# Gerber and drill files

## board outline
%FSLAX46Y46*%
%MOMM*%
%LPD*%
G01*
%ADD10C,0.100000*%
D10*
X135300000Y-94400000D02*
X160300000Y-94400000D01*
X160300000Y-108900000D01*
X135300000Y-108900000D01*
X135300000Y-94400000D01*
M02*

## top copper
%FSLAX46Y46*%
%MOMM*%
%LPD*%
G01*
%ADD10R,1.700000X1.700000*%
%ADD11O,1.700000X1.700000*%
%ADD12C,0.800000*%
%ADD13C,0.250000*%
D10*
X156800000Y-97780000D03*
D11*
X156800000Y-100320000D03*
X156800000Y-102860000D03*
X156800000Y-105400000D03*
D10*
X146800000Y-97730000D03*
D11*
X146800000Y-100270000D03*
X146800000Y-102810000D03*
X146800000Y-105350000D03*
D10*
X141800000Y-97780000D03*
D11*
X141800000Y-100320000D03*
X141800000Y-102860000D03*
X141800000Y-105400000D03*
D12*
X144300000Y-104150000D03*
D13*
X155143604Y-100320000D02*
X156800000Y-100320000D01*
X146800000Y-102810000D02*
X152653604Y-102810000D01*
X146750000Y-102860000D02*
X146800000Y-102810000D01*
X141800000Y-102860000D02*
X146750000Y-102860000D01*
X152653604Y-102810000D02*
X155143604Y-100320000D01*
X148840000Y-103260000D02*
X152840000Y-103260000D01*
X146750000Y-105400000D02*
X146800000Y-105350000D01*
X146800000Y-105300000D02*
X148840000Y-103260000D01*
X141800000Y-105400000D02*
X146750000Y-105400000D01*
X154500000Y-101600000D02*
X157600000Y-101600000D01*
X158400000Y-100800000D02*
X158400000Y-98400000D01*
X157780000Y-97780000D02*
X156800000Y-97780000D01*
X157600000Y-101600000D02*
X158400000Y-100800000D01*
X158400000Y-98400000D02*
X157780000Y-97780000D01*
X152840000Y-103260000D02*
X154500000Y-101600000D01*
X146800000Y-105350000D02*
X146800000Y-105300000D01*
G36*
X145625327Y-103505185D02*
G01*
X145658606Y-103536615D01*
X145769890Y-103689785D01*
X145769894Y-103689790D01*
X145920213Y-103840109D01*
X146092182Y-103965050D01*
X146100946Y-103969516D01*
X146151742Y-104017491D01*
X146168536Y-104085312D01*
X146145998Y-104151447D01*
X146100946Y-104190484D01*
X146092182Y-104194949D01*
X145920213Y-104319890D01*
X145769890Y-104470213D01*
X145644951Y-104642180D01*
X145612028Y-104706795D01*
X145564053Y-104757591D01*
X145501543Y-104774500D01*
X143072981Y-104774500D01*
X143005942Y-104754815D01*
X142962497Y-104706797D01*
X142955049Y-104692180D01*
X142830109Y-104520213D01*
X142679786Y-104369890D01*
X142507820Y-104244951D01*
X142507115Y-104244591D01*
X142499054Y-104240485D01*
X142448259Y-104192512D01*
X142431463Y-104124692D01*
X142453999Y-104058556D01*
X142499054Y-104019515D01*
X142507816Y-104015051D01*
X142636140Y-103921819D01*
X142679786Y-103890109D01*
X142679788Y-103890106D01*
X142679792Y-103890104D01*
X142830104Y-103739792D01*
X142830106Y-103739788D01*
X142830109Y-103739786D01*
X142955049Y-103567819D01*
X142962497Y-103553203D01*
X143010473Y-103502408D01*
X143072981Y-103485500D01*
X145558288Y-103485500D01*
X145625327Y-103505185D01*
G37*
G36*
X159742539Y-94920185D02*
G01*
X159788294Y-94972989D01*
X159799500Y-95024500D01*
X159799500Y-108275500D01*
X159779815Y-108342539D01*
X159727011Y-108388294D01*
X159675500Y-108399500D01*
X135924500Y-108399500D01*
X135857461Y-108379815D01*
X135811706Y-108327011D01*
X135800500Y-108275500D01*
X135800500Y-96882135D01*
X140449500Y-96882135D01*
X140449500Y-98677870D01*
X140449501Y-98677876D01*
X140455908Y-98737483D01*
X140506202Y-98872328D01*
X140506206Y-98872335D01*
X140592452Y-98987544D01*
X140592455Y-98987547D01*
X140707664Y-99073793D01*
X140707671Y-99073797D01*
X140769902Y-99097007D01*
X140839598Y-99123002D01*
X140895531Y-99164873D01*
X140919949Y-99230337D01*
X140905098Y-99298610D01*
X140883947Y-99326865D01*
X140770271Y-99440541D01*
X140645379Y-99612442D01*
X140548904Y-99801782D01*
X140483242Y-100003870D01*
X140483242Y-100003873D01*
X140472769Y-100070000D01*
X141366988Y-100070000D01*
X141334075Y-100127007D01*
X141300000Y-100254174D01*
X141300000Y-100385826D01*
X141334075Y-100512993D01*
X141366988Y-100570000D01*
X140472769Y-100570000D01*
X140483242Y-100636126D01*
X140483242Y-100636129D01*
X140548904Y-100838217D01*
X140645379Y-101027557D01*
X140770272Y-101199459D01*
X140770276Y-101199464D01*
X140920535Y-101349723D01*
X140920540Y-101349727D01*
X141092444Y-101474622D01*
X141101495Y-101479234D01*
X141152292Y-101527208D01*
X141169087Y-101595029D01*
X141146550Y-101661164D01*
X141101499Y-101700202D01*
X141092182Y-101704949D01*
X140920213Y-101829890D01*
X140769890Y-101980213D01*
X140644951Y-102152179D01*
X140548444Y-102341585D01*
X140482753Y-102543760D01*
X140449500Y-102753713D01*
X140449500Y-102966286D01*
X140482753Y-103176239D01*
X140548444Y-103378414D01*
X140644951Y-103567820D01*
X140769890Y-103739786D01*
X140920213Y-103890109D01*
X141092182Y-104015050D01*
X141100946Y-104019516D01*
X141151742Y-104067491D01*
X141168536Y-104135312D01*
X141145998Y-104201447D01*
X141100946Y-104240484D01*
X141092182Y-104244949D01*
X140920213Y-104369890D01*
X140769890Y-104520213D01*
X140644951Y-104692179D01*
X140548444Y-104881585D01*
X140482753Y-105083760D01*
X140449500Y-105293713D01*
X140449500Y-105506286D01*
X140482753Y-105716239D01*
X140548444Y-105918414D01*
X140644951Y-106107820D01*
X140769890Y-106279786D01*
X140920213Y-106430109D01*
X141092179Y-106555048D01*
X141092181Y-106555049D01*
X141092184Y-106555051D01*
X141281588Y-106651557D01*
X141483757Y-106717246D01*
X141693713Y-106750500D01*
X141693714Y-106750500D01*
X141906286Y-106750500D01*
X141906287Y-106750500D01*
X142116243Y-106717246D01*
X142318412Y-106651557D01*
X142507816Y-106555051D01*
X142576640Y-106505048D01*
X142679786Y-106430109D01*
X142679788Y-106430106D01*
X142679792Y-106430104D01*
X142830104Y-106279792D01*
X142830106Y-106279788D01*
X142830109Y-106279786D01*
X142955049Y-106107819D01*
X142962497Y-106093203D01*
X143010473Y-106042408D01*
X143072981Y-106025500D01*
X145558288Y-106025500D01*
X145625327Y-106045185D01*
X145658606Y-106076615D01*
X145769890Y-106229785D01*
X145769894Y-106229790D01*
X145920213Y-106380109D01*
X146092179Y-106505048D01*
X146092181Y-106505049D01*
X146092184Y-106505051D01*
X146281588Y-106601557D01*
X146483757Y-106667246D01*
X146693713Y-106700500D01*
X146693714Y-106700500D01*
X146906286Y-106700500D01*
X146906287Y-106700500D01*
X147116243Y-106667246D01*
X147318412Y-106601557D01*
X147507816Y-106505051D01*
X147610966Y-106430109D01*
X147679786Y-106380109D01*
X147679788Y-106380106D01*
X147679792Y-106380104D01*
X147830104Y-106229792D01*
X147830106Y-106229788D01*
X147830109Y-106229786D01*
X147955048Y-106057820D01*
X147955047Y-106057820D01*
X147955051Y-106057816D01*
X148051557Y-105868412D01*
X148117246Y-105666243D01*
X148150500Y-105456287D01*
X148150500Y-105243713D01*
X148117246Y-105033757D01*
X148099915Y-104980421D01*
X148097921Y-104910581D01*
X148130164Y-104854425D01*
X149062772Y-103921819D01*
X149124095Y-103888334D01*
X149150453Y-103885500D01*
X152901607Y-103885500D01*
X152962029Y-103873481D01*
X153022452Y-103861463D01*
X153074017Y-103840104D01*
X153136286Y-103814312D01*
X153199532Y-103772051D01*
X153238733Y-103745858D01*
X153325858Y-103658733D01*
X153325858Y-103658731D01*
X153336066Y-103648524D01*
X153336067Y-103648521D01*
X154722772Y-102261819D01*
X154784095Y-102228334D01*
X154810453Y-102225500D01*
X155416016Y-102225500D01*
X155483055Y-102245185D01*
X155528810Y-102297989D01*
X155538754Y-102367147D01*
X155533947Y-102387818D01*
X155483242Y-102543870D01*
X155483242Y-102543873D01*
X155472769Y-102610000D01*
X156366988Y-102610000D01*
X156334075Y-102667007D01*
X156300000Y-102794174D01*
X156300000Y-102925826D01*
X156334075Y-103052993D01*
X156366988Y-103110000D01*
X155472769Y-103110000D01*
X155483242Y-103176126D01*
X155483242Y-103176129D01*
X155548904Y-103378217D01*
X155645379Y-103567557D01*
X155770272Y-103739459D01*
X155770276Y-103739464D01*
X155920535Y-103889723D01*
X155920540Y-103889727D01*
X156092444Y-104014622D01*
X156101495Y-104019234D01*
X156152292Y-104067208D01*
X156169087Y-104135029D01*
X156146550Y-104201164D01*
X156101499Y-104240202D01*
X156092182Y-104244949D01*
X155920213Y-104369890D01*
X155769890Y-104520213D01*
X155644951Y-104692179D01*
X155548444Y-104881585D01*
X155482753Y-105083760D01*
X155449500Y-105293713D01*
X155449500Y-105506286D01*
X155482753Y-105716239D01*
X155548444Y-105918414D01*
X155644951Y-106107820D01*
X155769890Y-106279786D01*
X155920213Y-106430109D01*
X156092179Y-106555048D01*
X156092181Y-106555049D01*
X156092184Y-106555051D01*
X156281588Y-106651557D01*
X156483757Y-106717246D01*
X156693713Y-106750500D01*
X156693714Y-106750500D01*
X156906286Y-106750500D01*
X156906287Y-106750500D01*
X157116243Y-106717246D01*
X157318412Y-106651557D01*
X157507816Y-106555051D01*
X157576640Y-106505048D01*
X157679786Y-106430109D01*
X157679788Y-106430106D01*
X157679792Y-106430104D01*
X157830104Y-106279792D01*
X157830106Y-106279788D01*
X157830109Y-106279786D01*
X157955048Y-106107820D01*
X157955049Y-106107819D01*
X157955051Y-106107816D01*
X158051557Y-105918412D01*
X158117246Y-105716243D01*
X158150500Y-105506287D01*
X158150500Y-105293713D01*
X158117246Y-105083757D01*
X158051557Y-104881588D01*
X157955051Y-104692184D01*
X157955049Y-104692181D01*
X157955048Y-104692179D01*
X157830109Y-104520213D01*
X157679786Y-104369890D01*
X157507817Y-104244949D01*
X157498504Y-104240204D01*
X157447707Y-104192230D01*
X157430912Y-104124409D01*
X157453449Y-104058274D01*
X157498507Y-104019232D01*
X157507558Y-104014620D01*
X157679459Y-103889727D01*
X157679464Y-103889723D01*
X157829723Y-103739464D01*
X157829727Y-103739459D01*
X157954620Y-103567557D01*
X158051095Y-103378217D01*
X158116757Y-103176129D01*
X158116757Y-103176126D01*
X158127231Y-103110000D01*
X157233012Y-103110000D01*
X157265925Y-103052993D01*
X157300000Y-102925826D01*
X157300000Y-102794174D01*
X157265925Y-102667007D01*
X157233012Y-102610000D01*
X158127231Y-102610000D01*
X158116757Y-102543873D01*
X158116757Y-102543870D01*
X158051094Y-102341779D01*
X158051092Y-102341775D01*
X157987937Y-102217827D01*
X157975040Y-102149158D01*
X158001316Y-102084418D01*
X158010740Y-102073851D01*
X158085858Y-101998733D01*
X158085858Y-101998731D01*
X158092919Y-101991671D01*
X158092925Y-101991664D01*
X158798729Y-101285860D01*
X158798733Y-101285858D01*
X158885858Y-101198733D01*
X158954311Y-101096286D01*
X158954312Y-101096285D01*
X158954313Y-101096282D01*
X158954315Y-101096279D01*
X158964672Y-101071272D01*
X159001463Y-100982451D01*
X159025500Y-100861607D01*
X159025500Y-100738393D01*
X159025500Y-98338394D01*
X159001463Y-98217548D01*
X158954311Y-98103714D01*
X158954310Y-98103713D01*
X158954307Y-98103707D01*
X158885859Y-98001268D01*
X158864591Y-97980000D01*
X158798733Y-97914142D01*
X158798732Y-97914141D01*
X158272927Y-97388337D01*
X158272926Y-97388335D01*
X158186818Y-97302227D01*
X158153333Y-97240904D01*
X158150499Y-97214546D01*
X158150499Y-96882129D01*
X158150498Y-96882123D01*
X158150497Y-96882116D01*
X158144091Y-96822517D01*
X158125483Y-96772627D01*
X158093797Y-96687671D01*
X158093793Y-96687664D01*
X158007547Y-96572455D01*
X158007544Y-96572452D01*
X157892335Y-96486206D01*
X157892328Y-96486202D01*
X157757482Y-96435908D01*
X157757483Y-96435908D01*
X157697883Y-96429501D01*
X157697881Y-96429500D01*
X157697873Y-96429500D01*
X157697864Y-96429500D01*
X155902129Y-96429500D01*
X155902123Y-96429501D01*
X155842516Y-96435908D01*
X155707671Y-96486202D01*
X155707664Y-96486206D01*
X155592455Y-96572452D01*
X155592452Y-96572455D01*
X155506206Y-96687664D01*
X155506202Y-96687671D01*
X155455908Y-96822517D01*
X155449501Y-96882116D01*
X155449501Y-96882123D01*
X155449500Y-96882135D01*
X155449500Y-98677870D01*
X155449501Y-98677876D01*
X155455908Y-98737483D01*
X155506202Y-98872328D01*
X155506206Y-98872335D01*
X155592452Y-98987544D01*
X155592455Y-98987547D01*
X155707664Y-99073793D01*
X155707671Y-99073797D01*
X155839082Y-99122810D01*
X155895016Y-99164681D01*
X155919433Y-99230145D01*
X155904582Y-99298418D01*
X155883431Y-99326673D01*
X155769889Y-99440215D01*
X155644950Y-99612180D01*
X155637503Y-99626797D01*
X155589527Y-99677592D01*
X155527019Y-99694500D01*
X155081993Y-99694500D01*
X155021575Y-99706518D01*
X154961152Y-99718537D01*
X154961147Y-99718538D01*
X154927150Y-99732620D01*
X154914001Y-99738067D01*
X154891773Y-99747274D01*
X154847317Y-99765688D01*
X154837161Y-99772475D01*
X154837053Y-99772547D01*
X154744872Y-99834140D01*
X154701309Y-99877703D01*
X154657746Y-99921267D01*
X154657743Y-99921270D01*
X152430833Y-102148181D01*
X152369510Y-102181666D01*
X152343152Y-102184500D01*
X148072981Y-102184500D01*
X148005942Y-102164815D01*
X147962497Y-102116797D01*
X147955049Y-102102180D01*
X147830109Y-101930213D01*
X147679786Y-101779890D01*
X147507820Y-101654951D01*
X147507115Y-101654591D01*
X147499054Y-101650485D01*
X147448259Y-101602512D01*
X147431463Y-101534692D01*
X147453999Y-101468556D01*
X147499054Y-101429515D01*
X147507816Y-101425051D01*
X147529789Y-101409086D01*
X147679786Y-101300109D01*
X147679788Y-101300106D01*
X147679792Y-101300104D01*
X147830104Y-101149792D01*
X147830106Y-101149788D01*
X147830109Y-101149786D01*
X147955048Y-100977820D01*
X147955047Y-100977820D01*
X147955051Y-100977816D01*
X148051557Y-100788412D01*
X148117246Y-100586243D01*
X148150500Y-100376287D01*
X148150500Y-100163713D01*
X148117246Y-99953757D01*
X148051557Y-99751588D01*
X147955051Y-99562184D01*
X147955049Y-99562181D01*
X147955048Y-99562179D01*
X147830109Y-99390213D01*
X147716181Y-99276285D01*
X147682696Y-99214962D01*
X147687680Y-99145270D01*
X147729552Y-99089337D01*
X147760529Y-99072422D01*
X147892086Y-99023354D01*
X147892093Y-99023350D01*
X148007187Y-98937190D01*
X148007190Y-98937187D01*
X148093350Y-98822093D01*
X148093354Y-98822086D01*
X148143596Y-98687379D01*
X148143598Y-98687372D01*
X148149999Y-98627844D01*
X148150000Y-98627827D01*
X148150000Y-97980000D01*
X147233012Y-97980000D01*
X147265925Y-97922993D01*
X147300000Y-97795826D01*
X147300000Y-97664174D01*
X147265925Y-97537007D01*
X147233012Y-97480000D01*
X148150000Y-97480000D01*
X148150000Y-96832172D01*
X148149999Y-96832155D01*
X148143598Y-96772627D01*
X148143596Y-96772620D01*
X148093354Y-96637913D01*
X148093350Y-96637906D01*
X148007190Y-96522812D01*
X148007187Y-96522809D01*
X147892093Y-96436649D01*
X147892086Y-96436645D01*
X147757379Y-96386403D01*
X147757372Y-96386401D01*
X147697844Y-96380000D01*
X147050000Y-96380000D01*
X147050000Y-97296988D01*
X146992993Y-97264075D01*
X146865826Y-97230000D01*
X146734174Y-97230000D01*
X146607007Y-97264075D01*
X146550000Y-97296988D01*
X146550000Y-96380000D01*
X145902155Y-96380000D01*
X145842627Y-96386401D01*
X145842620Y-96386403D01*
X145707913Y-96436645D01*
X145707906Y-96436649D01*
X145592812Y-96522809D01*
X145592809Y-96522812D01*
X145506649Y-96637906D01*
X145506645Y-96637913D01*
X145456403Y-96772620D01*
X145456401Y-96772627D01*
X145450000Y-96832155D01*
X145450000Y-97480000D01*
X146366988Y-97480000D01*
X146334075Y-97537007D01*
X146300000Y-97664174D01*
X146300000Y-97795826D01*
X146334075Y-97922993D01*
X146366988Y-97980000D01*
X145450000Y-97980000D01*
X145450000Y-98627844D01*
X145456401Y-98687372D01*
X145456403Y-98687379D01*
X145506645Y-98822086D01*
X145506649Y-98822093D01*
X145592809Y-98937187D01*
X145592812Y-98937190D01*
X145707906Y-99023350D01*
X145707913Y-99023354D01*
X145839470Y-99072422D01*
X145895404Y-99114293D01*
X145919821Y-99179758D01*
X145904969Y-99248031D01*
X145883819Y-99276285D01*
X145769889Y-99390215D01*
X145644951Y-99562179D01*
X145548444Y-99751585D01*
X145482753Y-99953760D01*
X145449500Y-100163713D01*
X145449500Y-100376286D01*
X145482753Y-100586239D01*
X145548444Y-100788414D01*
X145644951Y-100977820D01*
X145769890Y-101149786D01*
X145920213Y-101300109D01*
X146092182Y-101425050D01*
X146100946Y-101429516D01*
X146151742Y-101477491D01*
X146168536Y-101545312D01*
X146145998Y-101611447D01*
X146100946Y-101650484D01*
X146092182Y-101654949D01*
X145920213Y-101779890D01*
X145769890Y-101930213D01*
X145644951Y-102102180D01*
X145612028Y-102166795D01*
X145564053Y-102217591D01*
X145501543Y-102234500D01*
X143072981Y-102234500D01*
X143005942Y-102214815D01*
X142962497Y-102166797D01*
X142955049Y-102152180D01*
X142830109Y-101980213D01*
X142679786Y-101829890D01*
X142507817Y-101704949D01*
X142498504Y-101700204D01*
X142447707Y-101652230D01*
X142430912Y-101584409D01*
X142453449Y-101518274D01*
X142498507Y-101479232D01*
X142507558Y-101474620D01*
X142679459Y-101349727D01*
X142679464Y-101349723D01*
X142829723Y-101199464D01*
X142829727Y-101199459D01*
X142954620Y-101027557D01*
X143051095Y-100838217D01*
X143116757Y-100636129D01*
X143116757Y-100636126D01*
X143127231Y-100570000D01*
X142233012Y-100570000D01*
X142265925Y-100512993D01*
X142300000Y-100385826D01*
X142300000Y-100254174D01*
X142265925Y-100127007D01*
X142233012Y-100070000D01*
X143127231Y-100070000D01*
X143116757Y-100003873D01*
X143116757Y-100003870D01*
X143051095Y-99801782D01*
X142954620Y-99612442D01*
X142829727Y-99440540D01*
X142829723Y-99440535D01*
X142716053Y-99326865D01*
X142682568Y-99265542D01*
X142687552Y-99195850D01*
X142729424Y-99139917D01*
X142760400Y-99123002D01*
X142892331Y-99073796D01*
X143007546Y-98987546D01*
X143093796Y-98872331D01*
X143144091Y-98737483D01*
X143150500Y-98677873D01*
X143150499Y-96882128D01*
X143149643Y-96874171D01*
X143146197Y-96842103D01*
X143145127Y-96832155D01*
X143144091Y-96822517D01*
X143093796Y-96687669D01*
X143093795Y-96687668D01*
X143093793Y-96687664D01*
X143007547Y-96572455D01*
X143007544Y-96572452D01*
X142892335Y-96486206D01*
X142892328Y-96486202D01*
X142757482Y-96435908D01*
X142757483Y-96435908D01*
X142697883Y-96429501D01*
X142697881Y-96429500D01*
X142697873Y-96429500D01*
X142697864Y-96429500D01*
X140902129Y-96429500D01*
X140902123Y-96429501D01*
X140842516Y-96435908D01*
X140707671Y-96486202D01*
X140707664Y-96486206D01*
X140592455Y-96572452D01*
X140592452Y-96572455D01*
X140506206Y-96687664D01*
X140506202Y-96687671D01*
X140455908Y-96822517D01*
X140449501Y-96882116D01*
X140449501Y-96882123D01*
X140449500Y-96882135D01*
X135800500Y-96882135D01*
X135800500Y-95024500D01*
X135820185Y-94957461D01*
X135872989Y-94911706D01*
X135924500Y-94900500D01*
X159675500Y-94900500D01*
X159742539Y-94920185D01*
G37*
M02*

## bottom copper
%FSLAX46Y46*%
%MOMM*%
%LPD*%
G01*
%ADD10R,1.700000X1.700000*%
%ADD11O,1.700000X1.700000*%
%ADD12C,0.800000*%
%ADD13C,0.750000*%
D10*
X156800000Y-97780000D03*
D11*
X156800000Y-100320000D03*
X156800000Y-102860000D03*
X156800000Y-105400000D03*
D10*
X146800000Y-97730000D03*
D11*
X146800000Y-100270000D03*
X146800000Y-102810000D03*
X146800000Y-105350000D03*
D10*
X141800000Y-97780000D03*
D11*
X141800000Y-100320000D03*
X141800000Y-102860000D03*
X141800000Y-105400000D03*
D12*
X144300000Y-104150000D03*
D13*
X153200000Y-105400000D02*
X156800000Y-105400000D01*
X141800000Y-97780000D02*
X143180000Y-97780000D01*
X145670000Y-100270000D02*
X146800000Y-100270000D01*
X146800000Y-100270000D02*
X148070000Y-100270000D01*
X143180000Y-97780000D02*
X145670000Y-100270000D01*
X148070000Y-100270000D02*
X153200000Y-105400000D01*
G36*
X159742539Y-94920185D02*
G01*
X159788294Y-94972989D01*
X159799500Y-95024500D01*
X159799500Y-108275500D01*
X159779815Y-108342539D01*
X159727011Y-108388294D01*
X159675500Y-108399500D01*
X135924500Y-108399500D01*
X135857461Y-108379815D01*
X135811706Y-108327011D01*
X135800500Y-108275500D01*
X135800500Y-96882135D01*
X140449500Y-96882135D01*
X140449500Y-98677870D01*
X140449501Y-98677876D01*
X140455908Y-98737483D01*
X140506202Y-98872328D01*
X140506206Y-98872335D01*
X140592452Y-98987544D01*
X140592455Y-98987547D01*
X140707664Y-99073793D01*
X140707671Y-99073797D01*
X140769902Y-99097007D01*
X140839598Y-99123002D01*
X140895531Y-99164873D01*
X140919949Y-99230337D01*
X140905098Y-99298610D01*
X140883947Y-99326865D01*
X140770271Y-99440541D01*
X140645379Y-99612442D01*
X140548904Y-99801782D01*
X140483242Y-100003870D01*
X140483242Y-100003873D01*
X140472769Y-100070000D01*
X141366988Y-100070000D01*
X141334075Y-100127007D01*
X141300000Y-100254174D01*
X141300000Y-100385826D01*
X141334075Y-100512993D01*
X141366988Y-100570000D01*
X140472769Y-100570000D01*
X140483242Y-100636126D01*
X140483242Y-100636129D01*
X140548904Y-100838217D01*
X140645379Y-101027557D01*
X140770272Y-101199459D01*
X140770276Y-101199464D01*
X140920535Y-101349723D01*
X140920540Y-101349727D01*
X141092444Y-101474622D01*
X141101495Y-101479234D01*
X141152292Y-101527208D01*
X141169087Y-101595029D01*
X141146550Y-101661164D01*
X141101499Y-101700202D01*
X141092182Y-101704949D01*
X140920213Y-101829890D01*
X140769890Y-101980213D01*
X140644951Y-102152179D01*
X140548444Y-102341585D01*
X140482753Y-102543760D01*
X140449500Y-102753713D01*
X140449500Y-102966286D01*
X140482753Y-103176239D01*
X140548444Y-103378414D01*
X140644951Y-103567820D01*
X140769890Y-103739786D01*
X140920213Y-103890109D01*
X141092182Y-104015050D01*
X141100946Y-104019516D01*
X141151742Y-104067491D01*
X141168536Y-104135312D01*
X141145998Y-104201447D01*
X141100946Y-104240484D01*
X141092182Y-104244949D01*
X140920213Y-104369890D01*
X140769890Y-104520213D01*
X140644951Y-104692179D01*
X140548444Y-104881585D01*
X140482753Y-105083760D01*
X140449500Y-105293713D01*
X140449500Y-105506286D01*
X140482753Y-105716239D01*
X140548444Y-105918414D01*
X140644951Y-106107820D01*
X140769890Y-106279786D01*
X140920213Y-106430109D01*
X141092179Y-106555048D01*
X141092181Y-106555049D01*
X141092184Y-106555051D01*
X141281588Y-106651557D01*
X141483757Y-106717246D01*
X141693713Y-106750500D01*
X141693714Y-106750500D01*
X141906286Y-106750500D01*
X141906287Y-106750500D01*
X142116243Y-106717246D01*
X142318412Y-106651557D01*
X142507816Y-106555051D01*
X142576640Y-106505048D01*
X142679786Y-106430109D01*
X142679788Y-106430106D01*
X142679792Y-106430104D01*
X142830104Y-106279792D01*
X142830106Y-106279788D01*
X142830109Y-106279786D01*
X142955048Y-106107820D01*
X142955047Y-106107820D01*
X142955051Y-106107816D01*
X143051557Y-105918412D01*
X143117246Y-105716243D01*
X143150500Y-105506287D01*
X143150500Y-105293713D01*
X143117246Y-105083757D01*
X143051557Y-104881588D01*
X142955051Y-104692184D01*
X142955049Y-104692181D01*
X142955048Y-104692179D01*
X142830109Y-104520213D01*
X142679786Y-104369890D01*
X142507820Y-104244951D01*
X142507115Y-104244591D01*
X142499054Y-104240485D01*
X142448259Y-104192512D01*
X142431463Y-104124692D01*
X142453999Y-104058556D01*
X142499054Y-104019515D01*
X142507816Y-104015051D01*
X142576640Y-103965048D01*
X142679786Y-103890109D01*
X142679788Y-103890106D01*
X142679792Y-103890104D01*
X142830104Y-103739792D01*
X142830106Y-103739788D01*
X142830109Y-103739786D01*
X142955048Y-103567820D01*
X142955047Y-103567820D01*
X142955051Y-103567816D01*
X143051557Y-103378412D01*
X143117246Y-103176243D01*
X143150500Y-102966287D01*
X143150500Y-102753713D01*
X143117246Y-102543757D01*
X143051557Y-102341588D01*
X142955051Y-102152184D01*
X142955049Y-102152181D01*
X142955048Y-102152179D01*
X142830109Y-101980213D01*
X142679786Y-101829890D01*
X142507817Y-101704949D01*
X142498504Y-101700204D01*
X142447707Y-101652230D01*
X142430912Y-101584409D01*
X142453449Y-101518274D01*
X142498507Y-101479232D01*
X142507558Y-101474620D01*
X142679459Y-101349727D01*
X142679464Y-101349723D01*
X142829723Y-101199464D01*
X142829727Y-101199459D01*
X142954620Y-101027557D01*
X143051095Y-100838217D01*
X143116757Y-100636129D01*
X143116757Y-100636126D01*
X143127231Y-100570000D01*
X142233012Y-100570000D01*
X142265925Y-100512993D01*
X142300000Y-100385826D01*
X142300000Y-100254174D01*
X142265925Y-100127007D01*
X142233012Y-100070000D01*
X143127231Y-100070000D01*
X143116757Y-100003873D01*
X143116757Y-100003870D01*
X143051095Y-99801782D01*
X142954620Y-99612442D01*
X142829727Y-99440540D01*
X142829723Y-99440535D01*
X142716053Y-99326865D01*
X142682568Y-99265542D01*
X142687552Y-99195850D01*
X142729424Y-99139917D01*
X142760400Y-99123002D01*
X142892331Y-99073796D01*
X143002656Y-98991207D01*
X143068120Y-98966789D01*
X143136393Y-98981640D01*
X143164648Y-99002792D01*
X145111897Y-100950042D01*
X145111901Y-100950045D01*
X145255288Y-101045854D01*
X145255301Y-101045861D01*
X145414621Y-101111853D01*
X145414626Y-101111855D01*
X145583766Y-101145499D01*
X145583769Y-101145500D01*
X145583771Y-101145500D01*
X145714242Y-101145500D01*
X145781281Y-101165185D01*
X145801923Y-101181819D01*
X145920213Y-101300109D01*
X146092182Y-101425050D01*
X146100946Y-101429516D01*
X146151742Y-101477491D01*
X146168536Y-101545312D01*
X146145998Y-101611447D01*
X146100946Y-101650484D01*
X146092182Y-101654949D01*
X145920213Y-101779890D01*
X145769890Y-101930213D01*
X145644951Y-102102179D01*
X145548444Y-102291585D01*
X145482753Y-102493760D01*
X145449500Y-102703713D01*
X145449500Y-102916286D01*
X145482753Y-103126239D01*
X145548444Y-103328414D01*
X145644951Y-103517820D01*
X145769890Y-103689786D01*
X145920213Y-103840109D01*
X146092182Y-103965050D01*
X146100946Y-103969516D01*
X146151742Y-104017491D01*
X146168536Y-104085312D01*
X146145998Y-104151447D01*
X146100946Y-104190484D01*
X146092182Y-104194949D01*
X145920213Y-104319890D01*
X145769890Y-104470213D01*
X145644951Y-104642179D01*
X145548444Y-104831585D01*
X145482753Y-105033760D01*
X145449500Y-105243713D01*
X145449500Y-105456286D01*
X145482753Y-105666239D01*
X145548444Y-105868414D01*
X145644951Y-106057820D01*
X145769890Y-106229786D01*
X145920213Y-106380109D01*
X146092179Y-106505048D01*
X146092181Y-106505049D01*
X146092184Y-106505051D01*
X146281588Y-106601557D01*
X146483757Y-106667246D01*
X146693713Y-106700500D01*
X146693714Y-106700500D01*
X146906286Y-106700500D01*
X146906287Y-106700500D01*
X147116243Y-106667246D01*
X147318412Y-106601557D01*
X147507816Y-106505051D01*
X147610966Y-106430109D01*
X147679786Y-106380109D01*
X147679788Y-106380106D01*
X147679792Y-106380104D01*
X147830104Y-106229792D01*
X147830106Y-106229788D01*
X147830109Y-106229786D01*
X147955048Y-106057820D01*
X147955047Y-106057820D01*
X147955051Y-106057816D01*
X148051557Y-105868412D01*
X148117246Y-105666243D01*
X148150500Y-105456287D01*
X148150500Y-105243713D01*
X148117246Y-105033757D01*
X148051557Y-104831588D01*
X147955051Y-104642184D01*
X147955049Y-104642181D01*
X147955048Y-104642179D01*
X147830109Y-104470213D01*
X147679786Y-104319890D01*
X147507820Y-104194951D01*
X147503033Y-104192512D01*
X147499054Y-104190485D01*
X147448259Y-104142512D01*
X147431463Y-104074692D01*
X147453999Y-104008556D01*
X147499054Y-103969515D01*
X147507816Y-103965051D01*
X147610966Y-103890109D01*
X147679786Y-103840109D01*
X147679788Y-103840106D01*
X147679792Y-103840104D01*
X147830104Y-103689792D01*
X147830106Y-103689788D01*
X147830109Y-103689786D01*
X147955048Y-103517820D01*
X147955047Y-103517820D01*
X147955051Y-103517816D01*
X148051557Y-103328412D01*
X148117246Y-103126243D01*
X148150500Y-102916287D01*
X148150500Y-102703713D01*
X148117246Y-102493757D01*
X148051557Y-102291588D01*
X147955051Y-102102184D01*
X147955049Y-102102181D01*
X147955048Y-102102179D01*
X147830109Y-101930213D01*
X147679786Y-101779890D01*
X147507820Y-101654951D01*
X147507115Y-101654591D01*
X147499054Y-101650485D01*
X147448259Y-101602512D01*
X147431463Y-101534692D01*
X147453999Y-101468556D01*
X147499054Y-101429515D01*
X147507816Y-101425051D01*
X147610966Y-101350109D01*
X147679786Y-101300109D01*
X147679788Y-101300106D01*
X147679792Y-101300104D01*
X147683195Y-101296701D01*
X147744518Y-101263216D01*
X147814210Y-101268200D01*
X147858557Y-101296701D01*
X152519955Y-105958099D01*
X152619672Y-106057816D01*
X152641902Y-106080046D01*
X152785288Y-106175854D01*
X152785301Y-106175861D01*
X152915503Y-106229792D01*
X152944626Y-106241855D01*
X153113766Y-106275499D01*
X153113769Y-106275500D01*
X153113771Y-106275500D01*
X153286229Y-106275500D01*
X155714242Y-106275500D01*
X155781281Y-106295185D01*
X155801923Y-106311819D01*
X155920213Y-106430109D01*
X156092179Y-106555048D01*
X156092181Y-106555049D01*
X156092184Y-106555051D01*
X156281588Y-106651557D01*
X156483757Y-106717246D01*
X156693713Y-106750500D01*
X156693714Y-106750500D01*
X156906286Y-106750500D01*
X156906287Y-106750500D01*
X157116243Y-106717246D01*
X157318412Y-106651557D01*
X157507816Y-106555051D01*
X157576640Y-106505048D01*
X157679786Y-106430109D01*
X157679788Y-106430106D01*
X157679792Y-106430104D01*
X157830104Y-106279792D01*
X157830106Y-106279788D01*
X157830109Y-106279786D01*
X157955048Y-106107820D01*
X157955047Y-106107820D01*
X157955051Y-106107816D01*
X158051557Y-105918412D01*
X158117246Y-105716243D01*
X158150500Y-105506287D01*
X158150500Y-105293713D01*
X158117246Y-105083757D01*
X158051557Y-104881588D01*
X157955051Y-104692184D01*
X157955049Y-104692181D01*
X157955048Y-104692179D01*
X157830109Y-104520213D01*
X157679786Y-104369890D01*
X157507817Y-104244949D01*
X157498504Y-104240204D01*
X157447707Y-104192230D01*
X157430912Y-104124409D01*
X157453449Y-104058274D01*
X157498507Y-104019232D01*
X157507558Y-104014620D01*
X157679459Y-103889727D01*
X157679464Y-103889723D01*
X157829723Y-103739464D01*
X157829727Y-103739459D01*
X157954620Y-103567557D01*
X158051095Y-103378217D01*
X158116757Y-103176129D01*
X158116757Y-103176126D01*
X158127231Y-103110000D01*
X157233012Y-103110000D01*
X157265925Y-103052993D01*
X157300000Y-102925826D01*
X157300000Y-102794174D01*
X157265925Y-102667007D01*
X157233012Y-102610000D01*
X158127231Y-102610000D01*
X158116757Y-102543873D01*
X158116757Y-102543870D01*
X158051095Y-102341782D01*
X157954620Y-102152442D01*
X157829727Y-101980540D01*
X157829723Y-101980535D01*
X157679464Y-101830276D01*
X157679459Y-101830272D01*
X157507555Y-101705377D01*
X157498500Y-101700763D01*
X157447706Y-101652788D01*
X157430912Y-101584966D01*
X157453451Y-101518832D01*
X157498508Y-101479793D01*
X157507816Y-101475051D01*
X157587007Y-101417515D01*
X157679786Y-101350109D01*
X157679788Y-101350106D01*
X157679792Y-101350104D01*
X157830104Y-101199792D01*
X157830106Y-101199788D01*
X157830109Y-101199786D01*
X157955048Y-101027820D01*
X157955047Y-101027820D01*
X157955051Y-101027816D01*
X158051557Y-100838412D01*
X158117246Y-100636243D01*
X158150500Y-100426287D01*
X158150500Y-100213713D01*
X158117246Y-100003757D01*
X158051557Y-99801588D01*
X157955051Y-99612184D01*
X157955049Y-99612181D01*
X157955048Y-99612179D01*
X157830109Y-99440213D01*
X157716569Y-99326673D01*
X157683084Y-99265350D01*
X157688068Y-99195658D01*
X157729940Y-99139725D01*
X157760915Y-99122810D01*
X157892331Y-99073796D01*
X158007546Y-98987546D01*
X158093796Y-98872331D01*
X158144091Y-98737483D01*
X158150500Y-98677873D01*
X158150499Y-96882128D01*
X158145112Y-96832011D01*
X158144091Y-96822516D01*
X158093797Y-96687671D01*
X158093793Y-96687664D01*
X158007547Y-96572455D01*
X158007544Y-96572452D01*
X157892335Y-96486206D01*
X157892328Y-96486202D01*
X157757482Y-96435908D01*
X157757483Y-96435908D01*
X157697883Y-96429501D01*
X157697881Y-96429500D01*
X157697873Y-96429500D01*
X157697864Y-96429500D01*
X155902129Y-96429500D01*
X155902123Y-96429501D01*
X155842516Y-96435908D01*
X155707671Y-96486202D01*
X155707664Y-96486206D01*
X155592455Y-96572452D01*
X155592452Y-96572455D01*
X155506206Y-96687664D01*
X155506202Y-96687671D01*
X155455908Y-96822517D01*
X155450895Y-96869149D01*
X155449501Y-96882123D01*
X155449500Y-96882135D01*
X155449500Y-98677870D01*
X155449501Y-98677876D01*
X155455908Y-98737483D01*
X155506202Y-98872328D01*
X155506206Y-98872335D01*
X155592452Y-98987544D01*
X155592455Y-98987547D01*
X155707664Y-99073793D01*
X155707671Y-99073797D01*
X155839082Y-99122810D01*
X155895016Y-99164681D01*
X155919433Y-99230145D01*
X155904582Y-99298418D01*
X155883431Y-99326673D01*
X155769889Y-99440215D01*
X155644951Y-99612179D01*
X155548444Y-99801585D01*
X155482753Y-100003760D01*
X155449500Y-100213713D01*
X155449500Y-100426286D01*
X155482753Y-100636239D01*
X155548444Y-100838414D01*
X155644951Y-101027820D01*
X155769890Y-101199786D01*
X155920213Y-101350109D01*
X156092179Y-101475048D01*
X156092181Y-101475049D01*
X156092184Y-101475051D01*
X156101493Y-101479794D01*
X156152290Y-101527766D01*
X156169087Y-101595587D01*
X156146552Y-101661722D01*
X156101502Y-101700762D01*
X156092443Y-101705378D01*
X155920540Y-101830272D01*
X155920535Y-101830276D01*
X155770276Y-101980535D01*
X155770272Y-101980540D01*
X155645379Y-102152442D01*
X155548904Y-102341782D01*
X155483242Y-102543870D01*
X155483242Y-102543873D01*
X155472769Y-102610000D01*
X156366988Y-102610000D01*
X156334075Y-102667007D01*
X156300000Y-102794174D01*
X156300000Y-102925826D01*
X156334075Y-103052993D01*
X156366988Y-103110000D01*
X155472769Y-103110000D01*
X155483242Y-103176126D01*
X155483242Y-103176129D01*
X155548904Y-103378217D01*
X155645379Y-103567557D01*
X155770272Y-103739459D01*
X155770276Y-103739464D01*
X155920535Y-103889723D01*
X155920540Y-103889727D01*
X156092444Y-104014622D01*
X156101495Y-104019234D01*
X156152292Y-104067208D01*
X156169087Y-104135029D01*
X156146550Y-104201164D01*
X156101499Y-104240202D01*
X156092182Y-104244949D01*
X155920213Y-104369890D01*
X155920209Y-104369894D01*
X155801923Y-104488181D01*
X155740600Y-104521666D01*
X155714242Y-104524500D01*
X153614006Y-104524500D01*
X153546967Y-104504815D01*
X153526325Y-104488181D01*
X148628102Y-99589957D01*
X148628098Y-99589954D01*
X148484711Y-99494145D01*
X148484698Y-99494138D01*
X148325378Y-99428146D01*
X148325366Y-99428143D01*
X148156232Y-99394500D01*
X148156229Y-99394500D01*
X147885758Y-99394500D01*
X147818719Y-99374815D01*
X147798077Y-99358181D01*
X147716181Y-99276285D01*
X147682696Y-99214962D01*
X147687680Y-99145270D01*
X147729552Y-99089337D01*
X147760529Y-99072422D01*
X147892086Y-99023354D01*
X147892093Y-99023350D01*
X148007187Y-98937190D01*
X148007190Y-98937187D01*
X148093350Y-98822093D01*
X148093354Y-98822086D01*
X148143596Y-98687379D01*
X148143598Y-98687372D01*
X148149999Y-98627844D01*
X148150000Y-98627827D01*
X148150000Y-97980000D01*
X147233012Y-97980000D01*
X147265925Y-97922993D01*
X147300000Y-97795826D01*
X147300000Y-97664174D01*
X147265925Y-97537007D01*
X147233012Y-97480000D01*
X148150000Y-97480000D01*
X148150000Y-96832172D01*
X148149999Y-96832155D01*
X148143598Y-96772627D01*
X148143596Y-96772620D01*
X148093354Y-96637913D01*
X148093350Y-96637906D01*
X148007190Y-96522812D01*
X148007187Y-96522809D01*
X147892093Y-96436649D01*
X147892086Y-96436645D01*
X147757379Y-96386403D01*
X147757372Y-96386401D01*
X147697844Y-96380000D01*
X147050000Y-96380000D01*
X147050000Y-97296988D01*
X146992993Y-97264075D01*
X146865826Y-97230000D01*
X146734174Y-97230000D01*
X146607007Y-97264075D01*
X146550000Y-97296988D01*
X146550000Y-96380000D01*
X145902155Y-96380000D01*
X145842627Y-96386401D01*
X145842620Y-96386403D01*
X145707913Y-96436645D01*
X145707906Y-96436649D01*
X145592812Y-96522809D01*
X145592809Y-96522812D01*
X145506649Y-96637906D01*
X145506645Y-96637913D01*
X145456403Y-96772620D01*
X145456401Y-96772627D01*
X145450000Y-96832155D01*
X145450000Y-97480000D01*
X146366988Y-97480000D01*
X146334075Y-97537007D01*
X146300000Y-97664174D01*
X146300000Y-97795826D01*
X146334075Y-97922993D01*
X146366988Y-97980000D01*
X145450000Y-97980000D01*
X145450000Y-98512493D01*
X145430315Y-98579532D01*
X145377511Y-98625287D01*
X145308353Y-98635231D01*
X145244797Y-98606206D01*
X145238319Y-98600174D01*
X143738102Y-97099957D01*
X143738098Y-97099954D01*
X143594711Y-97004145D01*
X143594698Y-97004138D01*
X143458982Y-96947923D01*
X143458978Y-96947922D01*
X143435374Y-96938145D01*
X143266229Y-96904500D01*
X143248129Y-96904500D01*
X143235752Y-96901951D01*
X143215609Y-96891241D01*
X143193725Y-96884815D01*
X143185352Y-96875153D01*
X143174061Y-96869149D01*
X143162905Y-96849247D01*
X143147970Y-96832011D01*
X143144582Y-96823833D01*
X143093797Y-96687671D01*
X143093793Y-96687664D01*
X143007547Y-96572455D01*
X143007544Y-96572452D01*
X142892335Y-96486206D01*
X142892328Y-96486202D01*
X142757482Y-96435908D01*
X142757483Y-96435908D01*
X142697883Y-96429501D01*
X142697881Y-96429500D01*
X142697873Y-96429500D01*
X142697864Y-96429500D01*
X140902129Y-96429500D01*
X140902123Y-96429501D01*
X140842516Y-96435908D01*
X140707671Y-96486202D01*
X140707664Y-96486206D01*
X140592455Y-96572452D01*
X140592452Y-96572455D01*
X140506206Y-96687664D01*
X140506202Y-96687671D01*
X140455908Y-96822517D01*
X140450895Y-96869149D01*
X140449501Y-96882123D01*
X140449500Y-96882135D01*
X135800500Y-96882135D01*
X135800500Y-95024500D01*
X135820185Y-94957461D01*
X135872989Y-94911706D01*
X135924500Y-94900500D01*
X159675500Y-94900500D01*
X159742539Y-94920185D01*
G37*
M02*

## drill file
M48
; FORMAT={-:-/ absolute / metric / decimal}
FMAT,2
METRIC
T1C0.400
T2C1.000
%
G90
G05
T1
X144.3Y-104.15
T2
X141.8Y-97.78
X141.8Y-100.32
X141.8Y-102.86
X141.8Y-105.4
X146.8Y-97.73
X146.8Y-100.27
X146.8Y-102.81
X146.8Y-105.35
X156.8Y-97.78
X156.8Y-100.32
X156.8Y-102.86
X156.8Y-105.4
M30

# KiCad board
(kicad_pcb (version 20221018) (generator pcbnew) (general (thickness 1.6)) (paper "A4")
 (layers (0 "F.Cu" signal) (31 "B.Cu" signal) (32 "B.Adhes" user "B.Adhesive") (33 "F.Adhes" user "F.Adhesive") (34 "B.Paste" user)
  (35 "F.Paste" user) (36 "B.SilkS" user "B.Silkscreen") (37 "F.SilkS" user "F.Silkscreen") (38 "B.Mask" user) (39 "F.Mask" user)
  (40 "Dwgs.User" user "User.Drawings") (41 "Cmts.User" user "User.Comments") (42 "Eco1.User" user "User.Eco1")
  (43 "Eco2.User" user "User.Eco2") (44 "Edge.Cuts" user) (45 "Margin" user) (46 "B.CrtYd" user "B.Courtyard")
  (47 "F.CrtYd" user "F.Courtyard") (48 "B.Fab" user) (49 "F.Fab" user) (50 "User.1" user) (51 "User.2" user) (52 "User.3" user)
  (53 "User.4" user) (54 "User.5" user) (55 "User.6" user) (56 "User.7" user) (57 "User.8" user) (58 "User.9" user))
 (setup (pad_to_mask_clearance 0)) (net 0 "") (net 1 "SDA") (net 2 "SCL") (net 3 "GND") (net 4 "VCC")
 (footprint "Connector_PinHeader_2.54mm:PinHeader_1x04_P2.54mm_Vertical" (layer "F.Cu") (at 156.8 97.78)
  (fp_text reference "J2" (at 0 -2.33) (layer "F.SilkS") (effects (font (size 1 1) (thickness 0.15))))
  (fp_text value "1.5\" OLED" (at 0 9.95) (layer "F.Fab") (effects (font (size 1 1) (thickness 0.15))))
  (pad "1" thru_hole rect (at 0 0) (size 1.7 1.7) (drill 1) (layers "*.Cu" "*.Mask") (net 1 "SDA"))
  (pad "2" thru_hole oval (at 0 2.54) (size 1.7 1.7) (drill 1) (layers "*.Cu" "*.Mask") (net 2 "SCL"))
  (pad "3" thru_hole oval (at 0 5.08) (size 1.7 1.7) (drill 1) (layers "*.Cu" "*.Mask") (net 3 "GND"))
  (pad "4" thru_hole oval (at 0 7.62) (size 1.7 1.7) (drill 1) (layers "*.Cu" "*.Mask") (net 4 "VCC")))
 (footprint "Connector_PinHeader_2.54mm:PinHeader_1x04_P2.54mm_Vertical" (layer "F.Cu") (at 146.8 97.73)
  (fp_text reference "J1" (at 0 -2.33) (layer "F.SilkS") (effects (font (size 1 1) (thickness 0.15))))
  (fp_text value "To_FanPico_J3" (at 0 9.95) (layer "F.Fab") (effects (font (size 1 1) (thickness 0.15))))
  (pad "1" thru_hole rect (at 0 0) (size 1.7 1.7) (drill 1) (layers "*.Cu" "*.Mask") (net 3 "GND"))
  (pad "2" thru_hole oval (at 0 2.54) (size 1.7 1.7) (drill 1) (layers "*.Cu" "*.Mask") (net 4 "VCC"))
  (pad "3" thru_hole oval (at 0 5.08) (size 1.7 1.7) (drill 1) (layers "*.Cu" "*.Mask") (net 2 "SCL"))
  (pad "4" thru_hole oval (at 0 7.62) (size 1.7 1.7) (drill 1) (layers "*.Cu" "*.Mask") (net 1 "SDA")))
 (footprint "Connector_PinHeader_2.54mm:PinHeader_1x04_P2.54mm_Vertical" (layer "F.Cu") (at 141.8 97.78)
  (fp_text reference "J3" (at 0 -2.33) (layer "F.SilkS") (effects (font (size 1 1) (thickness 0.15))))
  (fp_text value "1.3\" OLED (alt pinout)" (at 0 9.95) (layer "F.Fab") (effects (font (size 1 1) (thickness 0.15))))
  (pad "1" thru_hole rect (at 0 0) (size 1.7 1.7) (drill 1) (layers "*.Cu" "*.Mask") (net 4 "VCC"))
  (pad "2" thru_hole oval (at 0 2.54) (size 1.7 1.7) (drill 1) (layers "*.Cu" "*.Mask") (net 3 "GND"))
  (pad "3" thru_hole oval (at 0 5.08) (size 1.7 1.7) (drill 1) (layers "*.Cu" "*.Mask") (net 2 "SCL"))
  (pad "4" thru_hole oval (at 0 7.62) (size 1.7 1.7) (drill 1) (layers "*.Cu" "*.Mask") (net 1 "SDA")))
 (gr_rect (start 135.3 94.4) (end 160.3 108.9) (stroke (width 0.1) (type default)) (fill none) (layer "Edge.Cuts"))
 (via (at 144.3 104.15) (size 0.8) (drill 0.4) (layers "F.Cu" "B.Cu") (free) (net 3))
 (segment (start 153.2 105.4) (end 156.8 105.4) (width 0.75) (layer "B.Cu") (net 4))
 (segment (start 141.8 97.78) (end 143.18 97.78) (width 0.75) (layer "B.Cu") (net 4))
 (segment (start 145.67 100.27) (end 146.8 100.27) (width 0.75) (layer "B.Cu") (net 4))
 (segment (start 146.8 100.27) (end 148.07 100.27) (width 0.75) (layer "B.Cu") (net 4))
 (segment (start 143.18 97.78) (end 145.67 100.27) (width 0.75) (layer "B.Cu") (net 4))
 (segment (start 148.07 100.27) (end 153.2 105.4) (width 0.75) (layer "B.Cu") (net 4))
 (segment (start 155.143604 100.32) (end 156.8 100.32) (width 0.25) (layer "F.Cu") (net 2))
 (segment (start 146.8 102.81) (end 152.653604 102.81) (width 0.25) (layer "F.Cu") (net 2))
 (segment (start 146.75 102.86) (end 146.8 102.81) (width 0.25) (layer "F.Cu") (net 2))
 (segment (start 141.8 102.86) (end 146.75 102.86) (width 0.25) (layer "F.Cu") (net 2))
 (segment (start 152.653604 102.81) (end 155.143604 100.32) (width 0.25) (layer "F.Cu") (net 2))
 (segment (start 148.84 103.26) (end 152.84 103.26) (width 0.25) (layer "F.Cu") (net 1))
 (segment (start 146.75 105.4) (end 146.8 105.35) (width 0.25) (layer "F.Cu") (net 1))
 (segment (start 146.8 105.3) (end 148.84 103.26) (width 0.25) (layer "F.Cu") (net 1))
 (segment (start 141.8 105.4) (end 146.75 105.4) (width 0.25) (layer "F.Cu") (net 1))
 (segment (start 154.5 101.6) (end 157.6 101.6) (width 0.25) (layer "F.Cu") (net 1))
 (segment (start 158.4 100.8) (end 158.4 98.4) (width 0.25) (layer "F.Cu") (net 1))
 (segment (start 157.78 97.78) (end 156.8 97.78) (width 0.25) (layer "F.Cu") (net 1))
 (segment (start 157.6 101.6) (end 158.4 100.8) (width 0.25) (layer "F.Cu") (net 1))
 (segment (start 158.4 98.4) (end 157.78 97.78) (width 0.25) (layer "F.Cu") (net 1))
 (segment (start 152.84 103.26) (end 154.5 101.6) (width 0.25) (layer "F.Cu") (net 1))
 (segment (start 146.8 105.35) (end 146.8 105.3) (width 0.25) (layer "F.Cu") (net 1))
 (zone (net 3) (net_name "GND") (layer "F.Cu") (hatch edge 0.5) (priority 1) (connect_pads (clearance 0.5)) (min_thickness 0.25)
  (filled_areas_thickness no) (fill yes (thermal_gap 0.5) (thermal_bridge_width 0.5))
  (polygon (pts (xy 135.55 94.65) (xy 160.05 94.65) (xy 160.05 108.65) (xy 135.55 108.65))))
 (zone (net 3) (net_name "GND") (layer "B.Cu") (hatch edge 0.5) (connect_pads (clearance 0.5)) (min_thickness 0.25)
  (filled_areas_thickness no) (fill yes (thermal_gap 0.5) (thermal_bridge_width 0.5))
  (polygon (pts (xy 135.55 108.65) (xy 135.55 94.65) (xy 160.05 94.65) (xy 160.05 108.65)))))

